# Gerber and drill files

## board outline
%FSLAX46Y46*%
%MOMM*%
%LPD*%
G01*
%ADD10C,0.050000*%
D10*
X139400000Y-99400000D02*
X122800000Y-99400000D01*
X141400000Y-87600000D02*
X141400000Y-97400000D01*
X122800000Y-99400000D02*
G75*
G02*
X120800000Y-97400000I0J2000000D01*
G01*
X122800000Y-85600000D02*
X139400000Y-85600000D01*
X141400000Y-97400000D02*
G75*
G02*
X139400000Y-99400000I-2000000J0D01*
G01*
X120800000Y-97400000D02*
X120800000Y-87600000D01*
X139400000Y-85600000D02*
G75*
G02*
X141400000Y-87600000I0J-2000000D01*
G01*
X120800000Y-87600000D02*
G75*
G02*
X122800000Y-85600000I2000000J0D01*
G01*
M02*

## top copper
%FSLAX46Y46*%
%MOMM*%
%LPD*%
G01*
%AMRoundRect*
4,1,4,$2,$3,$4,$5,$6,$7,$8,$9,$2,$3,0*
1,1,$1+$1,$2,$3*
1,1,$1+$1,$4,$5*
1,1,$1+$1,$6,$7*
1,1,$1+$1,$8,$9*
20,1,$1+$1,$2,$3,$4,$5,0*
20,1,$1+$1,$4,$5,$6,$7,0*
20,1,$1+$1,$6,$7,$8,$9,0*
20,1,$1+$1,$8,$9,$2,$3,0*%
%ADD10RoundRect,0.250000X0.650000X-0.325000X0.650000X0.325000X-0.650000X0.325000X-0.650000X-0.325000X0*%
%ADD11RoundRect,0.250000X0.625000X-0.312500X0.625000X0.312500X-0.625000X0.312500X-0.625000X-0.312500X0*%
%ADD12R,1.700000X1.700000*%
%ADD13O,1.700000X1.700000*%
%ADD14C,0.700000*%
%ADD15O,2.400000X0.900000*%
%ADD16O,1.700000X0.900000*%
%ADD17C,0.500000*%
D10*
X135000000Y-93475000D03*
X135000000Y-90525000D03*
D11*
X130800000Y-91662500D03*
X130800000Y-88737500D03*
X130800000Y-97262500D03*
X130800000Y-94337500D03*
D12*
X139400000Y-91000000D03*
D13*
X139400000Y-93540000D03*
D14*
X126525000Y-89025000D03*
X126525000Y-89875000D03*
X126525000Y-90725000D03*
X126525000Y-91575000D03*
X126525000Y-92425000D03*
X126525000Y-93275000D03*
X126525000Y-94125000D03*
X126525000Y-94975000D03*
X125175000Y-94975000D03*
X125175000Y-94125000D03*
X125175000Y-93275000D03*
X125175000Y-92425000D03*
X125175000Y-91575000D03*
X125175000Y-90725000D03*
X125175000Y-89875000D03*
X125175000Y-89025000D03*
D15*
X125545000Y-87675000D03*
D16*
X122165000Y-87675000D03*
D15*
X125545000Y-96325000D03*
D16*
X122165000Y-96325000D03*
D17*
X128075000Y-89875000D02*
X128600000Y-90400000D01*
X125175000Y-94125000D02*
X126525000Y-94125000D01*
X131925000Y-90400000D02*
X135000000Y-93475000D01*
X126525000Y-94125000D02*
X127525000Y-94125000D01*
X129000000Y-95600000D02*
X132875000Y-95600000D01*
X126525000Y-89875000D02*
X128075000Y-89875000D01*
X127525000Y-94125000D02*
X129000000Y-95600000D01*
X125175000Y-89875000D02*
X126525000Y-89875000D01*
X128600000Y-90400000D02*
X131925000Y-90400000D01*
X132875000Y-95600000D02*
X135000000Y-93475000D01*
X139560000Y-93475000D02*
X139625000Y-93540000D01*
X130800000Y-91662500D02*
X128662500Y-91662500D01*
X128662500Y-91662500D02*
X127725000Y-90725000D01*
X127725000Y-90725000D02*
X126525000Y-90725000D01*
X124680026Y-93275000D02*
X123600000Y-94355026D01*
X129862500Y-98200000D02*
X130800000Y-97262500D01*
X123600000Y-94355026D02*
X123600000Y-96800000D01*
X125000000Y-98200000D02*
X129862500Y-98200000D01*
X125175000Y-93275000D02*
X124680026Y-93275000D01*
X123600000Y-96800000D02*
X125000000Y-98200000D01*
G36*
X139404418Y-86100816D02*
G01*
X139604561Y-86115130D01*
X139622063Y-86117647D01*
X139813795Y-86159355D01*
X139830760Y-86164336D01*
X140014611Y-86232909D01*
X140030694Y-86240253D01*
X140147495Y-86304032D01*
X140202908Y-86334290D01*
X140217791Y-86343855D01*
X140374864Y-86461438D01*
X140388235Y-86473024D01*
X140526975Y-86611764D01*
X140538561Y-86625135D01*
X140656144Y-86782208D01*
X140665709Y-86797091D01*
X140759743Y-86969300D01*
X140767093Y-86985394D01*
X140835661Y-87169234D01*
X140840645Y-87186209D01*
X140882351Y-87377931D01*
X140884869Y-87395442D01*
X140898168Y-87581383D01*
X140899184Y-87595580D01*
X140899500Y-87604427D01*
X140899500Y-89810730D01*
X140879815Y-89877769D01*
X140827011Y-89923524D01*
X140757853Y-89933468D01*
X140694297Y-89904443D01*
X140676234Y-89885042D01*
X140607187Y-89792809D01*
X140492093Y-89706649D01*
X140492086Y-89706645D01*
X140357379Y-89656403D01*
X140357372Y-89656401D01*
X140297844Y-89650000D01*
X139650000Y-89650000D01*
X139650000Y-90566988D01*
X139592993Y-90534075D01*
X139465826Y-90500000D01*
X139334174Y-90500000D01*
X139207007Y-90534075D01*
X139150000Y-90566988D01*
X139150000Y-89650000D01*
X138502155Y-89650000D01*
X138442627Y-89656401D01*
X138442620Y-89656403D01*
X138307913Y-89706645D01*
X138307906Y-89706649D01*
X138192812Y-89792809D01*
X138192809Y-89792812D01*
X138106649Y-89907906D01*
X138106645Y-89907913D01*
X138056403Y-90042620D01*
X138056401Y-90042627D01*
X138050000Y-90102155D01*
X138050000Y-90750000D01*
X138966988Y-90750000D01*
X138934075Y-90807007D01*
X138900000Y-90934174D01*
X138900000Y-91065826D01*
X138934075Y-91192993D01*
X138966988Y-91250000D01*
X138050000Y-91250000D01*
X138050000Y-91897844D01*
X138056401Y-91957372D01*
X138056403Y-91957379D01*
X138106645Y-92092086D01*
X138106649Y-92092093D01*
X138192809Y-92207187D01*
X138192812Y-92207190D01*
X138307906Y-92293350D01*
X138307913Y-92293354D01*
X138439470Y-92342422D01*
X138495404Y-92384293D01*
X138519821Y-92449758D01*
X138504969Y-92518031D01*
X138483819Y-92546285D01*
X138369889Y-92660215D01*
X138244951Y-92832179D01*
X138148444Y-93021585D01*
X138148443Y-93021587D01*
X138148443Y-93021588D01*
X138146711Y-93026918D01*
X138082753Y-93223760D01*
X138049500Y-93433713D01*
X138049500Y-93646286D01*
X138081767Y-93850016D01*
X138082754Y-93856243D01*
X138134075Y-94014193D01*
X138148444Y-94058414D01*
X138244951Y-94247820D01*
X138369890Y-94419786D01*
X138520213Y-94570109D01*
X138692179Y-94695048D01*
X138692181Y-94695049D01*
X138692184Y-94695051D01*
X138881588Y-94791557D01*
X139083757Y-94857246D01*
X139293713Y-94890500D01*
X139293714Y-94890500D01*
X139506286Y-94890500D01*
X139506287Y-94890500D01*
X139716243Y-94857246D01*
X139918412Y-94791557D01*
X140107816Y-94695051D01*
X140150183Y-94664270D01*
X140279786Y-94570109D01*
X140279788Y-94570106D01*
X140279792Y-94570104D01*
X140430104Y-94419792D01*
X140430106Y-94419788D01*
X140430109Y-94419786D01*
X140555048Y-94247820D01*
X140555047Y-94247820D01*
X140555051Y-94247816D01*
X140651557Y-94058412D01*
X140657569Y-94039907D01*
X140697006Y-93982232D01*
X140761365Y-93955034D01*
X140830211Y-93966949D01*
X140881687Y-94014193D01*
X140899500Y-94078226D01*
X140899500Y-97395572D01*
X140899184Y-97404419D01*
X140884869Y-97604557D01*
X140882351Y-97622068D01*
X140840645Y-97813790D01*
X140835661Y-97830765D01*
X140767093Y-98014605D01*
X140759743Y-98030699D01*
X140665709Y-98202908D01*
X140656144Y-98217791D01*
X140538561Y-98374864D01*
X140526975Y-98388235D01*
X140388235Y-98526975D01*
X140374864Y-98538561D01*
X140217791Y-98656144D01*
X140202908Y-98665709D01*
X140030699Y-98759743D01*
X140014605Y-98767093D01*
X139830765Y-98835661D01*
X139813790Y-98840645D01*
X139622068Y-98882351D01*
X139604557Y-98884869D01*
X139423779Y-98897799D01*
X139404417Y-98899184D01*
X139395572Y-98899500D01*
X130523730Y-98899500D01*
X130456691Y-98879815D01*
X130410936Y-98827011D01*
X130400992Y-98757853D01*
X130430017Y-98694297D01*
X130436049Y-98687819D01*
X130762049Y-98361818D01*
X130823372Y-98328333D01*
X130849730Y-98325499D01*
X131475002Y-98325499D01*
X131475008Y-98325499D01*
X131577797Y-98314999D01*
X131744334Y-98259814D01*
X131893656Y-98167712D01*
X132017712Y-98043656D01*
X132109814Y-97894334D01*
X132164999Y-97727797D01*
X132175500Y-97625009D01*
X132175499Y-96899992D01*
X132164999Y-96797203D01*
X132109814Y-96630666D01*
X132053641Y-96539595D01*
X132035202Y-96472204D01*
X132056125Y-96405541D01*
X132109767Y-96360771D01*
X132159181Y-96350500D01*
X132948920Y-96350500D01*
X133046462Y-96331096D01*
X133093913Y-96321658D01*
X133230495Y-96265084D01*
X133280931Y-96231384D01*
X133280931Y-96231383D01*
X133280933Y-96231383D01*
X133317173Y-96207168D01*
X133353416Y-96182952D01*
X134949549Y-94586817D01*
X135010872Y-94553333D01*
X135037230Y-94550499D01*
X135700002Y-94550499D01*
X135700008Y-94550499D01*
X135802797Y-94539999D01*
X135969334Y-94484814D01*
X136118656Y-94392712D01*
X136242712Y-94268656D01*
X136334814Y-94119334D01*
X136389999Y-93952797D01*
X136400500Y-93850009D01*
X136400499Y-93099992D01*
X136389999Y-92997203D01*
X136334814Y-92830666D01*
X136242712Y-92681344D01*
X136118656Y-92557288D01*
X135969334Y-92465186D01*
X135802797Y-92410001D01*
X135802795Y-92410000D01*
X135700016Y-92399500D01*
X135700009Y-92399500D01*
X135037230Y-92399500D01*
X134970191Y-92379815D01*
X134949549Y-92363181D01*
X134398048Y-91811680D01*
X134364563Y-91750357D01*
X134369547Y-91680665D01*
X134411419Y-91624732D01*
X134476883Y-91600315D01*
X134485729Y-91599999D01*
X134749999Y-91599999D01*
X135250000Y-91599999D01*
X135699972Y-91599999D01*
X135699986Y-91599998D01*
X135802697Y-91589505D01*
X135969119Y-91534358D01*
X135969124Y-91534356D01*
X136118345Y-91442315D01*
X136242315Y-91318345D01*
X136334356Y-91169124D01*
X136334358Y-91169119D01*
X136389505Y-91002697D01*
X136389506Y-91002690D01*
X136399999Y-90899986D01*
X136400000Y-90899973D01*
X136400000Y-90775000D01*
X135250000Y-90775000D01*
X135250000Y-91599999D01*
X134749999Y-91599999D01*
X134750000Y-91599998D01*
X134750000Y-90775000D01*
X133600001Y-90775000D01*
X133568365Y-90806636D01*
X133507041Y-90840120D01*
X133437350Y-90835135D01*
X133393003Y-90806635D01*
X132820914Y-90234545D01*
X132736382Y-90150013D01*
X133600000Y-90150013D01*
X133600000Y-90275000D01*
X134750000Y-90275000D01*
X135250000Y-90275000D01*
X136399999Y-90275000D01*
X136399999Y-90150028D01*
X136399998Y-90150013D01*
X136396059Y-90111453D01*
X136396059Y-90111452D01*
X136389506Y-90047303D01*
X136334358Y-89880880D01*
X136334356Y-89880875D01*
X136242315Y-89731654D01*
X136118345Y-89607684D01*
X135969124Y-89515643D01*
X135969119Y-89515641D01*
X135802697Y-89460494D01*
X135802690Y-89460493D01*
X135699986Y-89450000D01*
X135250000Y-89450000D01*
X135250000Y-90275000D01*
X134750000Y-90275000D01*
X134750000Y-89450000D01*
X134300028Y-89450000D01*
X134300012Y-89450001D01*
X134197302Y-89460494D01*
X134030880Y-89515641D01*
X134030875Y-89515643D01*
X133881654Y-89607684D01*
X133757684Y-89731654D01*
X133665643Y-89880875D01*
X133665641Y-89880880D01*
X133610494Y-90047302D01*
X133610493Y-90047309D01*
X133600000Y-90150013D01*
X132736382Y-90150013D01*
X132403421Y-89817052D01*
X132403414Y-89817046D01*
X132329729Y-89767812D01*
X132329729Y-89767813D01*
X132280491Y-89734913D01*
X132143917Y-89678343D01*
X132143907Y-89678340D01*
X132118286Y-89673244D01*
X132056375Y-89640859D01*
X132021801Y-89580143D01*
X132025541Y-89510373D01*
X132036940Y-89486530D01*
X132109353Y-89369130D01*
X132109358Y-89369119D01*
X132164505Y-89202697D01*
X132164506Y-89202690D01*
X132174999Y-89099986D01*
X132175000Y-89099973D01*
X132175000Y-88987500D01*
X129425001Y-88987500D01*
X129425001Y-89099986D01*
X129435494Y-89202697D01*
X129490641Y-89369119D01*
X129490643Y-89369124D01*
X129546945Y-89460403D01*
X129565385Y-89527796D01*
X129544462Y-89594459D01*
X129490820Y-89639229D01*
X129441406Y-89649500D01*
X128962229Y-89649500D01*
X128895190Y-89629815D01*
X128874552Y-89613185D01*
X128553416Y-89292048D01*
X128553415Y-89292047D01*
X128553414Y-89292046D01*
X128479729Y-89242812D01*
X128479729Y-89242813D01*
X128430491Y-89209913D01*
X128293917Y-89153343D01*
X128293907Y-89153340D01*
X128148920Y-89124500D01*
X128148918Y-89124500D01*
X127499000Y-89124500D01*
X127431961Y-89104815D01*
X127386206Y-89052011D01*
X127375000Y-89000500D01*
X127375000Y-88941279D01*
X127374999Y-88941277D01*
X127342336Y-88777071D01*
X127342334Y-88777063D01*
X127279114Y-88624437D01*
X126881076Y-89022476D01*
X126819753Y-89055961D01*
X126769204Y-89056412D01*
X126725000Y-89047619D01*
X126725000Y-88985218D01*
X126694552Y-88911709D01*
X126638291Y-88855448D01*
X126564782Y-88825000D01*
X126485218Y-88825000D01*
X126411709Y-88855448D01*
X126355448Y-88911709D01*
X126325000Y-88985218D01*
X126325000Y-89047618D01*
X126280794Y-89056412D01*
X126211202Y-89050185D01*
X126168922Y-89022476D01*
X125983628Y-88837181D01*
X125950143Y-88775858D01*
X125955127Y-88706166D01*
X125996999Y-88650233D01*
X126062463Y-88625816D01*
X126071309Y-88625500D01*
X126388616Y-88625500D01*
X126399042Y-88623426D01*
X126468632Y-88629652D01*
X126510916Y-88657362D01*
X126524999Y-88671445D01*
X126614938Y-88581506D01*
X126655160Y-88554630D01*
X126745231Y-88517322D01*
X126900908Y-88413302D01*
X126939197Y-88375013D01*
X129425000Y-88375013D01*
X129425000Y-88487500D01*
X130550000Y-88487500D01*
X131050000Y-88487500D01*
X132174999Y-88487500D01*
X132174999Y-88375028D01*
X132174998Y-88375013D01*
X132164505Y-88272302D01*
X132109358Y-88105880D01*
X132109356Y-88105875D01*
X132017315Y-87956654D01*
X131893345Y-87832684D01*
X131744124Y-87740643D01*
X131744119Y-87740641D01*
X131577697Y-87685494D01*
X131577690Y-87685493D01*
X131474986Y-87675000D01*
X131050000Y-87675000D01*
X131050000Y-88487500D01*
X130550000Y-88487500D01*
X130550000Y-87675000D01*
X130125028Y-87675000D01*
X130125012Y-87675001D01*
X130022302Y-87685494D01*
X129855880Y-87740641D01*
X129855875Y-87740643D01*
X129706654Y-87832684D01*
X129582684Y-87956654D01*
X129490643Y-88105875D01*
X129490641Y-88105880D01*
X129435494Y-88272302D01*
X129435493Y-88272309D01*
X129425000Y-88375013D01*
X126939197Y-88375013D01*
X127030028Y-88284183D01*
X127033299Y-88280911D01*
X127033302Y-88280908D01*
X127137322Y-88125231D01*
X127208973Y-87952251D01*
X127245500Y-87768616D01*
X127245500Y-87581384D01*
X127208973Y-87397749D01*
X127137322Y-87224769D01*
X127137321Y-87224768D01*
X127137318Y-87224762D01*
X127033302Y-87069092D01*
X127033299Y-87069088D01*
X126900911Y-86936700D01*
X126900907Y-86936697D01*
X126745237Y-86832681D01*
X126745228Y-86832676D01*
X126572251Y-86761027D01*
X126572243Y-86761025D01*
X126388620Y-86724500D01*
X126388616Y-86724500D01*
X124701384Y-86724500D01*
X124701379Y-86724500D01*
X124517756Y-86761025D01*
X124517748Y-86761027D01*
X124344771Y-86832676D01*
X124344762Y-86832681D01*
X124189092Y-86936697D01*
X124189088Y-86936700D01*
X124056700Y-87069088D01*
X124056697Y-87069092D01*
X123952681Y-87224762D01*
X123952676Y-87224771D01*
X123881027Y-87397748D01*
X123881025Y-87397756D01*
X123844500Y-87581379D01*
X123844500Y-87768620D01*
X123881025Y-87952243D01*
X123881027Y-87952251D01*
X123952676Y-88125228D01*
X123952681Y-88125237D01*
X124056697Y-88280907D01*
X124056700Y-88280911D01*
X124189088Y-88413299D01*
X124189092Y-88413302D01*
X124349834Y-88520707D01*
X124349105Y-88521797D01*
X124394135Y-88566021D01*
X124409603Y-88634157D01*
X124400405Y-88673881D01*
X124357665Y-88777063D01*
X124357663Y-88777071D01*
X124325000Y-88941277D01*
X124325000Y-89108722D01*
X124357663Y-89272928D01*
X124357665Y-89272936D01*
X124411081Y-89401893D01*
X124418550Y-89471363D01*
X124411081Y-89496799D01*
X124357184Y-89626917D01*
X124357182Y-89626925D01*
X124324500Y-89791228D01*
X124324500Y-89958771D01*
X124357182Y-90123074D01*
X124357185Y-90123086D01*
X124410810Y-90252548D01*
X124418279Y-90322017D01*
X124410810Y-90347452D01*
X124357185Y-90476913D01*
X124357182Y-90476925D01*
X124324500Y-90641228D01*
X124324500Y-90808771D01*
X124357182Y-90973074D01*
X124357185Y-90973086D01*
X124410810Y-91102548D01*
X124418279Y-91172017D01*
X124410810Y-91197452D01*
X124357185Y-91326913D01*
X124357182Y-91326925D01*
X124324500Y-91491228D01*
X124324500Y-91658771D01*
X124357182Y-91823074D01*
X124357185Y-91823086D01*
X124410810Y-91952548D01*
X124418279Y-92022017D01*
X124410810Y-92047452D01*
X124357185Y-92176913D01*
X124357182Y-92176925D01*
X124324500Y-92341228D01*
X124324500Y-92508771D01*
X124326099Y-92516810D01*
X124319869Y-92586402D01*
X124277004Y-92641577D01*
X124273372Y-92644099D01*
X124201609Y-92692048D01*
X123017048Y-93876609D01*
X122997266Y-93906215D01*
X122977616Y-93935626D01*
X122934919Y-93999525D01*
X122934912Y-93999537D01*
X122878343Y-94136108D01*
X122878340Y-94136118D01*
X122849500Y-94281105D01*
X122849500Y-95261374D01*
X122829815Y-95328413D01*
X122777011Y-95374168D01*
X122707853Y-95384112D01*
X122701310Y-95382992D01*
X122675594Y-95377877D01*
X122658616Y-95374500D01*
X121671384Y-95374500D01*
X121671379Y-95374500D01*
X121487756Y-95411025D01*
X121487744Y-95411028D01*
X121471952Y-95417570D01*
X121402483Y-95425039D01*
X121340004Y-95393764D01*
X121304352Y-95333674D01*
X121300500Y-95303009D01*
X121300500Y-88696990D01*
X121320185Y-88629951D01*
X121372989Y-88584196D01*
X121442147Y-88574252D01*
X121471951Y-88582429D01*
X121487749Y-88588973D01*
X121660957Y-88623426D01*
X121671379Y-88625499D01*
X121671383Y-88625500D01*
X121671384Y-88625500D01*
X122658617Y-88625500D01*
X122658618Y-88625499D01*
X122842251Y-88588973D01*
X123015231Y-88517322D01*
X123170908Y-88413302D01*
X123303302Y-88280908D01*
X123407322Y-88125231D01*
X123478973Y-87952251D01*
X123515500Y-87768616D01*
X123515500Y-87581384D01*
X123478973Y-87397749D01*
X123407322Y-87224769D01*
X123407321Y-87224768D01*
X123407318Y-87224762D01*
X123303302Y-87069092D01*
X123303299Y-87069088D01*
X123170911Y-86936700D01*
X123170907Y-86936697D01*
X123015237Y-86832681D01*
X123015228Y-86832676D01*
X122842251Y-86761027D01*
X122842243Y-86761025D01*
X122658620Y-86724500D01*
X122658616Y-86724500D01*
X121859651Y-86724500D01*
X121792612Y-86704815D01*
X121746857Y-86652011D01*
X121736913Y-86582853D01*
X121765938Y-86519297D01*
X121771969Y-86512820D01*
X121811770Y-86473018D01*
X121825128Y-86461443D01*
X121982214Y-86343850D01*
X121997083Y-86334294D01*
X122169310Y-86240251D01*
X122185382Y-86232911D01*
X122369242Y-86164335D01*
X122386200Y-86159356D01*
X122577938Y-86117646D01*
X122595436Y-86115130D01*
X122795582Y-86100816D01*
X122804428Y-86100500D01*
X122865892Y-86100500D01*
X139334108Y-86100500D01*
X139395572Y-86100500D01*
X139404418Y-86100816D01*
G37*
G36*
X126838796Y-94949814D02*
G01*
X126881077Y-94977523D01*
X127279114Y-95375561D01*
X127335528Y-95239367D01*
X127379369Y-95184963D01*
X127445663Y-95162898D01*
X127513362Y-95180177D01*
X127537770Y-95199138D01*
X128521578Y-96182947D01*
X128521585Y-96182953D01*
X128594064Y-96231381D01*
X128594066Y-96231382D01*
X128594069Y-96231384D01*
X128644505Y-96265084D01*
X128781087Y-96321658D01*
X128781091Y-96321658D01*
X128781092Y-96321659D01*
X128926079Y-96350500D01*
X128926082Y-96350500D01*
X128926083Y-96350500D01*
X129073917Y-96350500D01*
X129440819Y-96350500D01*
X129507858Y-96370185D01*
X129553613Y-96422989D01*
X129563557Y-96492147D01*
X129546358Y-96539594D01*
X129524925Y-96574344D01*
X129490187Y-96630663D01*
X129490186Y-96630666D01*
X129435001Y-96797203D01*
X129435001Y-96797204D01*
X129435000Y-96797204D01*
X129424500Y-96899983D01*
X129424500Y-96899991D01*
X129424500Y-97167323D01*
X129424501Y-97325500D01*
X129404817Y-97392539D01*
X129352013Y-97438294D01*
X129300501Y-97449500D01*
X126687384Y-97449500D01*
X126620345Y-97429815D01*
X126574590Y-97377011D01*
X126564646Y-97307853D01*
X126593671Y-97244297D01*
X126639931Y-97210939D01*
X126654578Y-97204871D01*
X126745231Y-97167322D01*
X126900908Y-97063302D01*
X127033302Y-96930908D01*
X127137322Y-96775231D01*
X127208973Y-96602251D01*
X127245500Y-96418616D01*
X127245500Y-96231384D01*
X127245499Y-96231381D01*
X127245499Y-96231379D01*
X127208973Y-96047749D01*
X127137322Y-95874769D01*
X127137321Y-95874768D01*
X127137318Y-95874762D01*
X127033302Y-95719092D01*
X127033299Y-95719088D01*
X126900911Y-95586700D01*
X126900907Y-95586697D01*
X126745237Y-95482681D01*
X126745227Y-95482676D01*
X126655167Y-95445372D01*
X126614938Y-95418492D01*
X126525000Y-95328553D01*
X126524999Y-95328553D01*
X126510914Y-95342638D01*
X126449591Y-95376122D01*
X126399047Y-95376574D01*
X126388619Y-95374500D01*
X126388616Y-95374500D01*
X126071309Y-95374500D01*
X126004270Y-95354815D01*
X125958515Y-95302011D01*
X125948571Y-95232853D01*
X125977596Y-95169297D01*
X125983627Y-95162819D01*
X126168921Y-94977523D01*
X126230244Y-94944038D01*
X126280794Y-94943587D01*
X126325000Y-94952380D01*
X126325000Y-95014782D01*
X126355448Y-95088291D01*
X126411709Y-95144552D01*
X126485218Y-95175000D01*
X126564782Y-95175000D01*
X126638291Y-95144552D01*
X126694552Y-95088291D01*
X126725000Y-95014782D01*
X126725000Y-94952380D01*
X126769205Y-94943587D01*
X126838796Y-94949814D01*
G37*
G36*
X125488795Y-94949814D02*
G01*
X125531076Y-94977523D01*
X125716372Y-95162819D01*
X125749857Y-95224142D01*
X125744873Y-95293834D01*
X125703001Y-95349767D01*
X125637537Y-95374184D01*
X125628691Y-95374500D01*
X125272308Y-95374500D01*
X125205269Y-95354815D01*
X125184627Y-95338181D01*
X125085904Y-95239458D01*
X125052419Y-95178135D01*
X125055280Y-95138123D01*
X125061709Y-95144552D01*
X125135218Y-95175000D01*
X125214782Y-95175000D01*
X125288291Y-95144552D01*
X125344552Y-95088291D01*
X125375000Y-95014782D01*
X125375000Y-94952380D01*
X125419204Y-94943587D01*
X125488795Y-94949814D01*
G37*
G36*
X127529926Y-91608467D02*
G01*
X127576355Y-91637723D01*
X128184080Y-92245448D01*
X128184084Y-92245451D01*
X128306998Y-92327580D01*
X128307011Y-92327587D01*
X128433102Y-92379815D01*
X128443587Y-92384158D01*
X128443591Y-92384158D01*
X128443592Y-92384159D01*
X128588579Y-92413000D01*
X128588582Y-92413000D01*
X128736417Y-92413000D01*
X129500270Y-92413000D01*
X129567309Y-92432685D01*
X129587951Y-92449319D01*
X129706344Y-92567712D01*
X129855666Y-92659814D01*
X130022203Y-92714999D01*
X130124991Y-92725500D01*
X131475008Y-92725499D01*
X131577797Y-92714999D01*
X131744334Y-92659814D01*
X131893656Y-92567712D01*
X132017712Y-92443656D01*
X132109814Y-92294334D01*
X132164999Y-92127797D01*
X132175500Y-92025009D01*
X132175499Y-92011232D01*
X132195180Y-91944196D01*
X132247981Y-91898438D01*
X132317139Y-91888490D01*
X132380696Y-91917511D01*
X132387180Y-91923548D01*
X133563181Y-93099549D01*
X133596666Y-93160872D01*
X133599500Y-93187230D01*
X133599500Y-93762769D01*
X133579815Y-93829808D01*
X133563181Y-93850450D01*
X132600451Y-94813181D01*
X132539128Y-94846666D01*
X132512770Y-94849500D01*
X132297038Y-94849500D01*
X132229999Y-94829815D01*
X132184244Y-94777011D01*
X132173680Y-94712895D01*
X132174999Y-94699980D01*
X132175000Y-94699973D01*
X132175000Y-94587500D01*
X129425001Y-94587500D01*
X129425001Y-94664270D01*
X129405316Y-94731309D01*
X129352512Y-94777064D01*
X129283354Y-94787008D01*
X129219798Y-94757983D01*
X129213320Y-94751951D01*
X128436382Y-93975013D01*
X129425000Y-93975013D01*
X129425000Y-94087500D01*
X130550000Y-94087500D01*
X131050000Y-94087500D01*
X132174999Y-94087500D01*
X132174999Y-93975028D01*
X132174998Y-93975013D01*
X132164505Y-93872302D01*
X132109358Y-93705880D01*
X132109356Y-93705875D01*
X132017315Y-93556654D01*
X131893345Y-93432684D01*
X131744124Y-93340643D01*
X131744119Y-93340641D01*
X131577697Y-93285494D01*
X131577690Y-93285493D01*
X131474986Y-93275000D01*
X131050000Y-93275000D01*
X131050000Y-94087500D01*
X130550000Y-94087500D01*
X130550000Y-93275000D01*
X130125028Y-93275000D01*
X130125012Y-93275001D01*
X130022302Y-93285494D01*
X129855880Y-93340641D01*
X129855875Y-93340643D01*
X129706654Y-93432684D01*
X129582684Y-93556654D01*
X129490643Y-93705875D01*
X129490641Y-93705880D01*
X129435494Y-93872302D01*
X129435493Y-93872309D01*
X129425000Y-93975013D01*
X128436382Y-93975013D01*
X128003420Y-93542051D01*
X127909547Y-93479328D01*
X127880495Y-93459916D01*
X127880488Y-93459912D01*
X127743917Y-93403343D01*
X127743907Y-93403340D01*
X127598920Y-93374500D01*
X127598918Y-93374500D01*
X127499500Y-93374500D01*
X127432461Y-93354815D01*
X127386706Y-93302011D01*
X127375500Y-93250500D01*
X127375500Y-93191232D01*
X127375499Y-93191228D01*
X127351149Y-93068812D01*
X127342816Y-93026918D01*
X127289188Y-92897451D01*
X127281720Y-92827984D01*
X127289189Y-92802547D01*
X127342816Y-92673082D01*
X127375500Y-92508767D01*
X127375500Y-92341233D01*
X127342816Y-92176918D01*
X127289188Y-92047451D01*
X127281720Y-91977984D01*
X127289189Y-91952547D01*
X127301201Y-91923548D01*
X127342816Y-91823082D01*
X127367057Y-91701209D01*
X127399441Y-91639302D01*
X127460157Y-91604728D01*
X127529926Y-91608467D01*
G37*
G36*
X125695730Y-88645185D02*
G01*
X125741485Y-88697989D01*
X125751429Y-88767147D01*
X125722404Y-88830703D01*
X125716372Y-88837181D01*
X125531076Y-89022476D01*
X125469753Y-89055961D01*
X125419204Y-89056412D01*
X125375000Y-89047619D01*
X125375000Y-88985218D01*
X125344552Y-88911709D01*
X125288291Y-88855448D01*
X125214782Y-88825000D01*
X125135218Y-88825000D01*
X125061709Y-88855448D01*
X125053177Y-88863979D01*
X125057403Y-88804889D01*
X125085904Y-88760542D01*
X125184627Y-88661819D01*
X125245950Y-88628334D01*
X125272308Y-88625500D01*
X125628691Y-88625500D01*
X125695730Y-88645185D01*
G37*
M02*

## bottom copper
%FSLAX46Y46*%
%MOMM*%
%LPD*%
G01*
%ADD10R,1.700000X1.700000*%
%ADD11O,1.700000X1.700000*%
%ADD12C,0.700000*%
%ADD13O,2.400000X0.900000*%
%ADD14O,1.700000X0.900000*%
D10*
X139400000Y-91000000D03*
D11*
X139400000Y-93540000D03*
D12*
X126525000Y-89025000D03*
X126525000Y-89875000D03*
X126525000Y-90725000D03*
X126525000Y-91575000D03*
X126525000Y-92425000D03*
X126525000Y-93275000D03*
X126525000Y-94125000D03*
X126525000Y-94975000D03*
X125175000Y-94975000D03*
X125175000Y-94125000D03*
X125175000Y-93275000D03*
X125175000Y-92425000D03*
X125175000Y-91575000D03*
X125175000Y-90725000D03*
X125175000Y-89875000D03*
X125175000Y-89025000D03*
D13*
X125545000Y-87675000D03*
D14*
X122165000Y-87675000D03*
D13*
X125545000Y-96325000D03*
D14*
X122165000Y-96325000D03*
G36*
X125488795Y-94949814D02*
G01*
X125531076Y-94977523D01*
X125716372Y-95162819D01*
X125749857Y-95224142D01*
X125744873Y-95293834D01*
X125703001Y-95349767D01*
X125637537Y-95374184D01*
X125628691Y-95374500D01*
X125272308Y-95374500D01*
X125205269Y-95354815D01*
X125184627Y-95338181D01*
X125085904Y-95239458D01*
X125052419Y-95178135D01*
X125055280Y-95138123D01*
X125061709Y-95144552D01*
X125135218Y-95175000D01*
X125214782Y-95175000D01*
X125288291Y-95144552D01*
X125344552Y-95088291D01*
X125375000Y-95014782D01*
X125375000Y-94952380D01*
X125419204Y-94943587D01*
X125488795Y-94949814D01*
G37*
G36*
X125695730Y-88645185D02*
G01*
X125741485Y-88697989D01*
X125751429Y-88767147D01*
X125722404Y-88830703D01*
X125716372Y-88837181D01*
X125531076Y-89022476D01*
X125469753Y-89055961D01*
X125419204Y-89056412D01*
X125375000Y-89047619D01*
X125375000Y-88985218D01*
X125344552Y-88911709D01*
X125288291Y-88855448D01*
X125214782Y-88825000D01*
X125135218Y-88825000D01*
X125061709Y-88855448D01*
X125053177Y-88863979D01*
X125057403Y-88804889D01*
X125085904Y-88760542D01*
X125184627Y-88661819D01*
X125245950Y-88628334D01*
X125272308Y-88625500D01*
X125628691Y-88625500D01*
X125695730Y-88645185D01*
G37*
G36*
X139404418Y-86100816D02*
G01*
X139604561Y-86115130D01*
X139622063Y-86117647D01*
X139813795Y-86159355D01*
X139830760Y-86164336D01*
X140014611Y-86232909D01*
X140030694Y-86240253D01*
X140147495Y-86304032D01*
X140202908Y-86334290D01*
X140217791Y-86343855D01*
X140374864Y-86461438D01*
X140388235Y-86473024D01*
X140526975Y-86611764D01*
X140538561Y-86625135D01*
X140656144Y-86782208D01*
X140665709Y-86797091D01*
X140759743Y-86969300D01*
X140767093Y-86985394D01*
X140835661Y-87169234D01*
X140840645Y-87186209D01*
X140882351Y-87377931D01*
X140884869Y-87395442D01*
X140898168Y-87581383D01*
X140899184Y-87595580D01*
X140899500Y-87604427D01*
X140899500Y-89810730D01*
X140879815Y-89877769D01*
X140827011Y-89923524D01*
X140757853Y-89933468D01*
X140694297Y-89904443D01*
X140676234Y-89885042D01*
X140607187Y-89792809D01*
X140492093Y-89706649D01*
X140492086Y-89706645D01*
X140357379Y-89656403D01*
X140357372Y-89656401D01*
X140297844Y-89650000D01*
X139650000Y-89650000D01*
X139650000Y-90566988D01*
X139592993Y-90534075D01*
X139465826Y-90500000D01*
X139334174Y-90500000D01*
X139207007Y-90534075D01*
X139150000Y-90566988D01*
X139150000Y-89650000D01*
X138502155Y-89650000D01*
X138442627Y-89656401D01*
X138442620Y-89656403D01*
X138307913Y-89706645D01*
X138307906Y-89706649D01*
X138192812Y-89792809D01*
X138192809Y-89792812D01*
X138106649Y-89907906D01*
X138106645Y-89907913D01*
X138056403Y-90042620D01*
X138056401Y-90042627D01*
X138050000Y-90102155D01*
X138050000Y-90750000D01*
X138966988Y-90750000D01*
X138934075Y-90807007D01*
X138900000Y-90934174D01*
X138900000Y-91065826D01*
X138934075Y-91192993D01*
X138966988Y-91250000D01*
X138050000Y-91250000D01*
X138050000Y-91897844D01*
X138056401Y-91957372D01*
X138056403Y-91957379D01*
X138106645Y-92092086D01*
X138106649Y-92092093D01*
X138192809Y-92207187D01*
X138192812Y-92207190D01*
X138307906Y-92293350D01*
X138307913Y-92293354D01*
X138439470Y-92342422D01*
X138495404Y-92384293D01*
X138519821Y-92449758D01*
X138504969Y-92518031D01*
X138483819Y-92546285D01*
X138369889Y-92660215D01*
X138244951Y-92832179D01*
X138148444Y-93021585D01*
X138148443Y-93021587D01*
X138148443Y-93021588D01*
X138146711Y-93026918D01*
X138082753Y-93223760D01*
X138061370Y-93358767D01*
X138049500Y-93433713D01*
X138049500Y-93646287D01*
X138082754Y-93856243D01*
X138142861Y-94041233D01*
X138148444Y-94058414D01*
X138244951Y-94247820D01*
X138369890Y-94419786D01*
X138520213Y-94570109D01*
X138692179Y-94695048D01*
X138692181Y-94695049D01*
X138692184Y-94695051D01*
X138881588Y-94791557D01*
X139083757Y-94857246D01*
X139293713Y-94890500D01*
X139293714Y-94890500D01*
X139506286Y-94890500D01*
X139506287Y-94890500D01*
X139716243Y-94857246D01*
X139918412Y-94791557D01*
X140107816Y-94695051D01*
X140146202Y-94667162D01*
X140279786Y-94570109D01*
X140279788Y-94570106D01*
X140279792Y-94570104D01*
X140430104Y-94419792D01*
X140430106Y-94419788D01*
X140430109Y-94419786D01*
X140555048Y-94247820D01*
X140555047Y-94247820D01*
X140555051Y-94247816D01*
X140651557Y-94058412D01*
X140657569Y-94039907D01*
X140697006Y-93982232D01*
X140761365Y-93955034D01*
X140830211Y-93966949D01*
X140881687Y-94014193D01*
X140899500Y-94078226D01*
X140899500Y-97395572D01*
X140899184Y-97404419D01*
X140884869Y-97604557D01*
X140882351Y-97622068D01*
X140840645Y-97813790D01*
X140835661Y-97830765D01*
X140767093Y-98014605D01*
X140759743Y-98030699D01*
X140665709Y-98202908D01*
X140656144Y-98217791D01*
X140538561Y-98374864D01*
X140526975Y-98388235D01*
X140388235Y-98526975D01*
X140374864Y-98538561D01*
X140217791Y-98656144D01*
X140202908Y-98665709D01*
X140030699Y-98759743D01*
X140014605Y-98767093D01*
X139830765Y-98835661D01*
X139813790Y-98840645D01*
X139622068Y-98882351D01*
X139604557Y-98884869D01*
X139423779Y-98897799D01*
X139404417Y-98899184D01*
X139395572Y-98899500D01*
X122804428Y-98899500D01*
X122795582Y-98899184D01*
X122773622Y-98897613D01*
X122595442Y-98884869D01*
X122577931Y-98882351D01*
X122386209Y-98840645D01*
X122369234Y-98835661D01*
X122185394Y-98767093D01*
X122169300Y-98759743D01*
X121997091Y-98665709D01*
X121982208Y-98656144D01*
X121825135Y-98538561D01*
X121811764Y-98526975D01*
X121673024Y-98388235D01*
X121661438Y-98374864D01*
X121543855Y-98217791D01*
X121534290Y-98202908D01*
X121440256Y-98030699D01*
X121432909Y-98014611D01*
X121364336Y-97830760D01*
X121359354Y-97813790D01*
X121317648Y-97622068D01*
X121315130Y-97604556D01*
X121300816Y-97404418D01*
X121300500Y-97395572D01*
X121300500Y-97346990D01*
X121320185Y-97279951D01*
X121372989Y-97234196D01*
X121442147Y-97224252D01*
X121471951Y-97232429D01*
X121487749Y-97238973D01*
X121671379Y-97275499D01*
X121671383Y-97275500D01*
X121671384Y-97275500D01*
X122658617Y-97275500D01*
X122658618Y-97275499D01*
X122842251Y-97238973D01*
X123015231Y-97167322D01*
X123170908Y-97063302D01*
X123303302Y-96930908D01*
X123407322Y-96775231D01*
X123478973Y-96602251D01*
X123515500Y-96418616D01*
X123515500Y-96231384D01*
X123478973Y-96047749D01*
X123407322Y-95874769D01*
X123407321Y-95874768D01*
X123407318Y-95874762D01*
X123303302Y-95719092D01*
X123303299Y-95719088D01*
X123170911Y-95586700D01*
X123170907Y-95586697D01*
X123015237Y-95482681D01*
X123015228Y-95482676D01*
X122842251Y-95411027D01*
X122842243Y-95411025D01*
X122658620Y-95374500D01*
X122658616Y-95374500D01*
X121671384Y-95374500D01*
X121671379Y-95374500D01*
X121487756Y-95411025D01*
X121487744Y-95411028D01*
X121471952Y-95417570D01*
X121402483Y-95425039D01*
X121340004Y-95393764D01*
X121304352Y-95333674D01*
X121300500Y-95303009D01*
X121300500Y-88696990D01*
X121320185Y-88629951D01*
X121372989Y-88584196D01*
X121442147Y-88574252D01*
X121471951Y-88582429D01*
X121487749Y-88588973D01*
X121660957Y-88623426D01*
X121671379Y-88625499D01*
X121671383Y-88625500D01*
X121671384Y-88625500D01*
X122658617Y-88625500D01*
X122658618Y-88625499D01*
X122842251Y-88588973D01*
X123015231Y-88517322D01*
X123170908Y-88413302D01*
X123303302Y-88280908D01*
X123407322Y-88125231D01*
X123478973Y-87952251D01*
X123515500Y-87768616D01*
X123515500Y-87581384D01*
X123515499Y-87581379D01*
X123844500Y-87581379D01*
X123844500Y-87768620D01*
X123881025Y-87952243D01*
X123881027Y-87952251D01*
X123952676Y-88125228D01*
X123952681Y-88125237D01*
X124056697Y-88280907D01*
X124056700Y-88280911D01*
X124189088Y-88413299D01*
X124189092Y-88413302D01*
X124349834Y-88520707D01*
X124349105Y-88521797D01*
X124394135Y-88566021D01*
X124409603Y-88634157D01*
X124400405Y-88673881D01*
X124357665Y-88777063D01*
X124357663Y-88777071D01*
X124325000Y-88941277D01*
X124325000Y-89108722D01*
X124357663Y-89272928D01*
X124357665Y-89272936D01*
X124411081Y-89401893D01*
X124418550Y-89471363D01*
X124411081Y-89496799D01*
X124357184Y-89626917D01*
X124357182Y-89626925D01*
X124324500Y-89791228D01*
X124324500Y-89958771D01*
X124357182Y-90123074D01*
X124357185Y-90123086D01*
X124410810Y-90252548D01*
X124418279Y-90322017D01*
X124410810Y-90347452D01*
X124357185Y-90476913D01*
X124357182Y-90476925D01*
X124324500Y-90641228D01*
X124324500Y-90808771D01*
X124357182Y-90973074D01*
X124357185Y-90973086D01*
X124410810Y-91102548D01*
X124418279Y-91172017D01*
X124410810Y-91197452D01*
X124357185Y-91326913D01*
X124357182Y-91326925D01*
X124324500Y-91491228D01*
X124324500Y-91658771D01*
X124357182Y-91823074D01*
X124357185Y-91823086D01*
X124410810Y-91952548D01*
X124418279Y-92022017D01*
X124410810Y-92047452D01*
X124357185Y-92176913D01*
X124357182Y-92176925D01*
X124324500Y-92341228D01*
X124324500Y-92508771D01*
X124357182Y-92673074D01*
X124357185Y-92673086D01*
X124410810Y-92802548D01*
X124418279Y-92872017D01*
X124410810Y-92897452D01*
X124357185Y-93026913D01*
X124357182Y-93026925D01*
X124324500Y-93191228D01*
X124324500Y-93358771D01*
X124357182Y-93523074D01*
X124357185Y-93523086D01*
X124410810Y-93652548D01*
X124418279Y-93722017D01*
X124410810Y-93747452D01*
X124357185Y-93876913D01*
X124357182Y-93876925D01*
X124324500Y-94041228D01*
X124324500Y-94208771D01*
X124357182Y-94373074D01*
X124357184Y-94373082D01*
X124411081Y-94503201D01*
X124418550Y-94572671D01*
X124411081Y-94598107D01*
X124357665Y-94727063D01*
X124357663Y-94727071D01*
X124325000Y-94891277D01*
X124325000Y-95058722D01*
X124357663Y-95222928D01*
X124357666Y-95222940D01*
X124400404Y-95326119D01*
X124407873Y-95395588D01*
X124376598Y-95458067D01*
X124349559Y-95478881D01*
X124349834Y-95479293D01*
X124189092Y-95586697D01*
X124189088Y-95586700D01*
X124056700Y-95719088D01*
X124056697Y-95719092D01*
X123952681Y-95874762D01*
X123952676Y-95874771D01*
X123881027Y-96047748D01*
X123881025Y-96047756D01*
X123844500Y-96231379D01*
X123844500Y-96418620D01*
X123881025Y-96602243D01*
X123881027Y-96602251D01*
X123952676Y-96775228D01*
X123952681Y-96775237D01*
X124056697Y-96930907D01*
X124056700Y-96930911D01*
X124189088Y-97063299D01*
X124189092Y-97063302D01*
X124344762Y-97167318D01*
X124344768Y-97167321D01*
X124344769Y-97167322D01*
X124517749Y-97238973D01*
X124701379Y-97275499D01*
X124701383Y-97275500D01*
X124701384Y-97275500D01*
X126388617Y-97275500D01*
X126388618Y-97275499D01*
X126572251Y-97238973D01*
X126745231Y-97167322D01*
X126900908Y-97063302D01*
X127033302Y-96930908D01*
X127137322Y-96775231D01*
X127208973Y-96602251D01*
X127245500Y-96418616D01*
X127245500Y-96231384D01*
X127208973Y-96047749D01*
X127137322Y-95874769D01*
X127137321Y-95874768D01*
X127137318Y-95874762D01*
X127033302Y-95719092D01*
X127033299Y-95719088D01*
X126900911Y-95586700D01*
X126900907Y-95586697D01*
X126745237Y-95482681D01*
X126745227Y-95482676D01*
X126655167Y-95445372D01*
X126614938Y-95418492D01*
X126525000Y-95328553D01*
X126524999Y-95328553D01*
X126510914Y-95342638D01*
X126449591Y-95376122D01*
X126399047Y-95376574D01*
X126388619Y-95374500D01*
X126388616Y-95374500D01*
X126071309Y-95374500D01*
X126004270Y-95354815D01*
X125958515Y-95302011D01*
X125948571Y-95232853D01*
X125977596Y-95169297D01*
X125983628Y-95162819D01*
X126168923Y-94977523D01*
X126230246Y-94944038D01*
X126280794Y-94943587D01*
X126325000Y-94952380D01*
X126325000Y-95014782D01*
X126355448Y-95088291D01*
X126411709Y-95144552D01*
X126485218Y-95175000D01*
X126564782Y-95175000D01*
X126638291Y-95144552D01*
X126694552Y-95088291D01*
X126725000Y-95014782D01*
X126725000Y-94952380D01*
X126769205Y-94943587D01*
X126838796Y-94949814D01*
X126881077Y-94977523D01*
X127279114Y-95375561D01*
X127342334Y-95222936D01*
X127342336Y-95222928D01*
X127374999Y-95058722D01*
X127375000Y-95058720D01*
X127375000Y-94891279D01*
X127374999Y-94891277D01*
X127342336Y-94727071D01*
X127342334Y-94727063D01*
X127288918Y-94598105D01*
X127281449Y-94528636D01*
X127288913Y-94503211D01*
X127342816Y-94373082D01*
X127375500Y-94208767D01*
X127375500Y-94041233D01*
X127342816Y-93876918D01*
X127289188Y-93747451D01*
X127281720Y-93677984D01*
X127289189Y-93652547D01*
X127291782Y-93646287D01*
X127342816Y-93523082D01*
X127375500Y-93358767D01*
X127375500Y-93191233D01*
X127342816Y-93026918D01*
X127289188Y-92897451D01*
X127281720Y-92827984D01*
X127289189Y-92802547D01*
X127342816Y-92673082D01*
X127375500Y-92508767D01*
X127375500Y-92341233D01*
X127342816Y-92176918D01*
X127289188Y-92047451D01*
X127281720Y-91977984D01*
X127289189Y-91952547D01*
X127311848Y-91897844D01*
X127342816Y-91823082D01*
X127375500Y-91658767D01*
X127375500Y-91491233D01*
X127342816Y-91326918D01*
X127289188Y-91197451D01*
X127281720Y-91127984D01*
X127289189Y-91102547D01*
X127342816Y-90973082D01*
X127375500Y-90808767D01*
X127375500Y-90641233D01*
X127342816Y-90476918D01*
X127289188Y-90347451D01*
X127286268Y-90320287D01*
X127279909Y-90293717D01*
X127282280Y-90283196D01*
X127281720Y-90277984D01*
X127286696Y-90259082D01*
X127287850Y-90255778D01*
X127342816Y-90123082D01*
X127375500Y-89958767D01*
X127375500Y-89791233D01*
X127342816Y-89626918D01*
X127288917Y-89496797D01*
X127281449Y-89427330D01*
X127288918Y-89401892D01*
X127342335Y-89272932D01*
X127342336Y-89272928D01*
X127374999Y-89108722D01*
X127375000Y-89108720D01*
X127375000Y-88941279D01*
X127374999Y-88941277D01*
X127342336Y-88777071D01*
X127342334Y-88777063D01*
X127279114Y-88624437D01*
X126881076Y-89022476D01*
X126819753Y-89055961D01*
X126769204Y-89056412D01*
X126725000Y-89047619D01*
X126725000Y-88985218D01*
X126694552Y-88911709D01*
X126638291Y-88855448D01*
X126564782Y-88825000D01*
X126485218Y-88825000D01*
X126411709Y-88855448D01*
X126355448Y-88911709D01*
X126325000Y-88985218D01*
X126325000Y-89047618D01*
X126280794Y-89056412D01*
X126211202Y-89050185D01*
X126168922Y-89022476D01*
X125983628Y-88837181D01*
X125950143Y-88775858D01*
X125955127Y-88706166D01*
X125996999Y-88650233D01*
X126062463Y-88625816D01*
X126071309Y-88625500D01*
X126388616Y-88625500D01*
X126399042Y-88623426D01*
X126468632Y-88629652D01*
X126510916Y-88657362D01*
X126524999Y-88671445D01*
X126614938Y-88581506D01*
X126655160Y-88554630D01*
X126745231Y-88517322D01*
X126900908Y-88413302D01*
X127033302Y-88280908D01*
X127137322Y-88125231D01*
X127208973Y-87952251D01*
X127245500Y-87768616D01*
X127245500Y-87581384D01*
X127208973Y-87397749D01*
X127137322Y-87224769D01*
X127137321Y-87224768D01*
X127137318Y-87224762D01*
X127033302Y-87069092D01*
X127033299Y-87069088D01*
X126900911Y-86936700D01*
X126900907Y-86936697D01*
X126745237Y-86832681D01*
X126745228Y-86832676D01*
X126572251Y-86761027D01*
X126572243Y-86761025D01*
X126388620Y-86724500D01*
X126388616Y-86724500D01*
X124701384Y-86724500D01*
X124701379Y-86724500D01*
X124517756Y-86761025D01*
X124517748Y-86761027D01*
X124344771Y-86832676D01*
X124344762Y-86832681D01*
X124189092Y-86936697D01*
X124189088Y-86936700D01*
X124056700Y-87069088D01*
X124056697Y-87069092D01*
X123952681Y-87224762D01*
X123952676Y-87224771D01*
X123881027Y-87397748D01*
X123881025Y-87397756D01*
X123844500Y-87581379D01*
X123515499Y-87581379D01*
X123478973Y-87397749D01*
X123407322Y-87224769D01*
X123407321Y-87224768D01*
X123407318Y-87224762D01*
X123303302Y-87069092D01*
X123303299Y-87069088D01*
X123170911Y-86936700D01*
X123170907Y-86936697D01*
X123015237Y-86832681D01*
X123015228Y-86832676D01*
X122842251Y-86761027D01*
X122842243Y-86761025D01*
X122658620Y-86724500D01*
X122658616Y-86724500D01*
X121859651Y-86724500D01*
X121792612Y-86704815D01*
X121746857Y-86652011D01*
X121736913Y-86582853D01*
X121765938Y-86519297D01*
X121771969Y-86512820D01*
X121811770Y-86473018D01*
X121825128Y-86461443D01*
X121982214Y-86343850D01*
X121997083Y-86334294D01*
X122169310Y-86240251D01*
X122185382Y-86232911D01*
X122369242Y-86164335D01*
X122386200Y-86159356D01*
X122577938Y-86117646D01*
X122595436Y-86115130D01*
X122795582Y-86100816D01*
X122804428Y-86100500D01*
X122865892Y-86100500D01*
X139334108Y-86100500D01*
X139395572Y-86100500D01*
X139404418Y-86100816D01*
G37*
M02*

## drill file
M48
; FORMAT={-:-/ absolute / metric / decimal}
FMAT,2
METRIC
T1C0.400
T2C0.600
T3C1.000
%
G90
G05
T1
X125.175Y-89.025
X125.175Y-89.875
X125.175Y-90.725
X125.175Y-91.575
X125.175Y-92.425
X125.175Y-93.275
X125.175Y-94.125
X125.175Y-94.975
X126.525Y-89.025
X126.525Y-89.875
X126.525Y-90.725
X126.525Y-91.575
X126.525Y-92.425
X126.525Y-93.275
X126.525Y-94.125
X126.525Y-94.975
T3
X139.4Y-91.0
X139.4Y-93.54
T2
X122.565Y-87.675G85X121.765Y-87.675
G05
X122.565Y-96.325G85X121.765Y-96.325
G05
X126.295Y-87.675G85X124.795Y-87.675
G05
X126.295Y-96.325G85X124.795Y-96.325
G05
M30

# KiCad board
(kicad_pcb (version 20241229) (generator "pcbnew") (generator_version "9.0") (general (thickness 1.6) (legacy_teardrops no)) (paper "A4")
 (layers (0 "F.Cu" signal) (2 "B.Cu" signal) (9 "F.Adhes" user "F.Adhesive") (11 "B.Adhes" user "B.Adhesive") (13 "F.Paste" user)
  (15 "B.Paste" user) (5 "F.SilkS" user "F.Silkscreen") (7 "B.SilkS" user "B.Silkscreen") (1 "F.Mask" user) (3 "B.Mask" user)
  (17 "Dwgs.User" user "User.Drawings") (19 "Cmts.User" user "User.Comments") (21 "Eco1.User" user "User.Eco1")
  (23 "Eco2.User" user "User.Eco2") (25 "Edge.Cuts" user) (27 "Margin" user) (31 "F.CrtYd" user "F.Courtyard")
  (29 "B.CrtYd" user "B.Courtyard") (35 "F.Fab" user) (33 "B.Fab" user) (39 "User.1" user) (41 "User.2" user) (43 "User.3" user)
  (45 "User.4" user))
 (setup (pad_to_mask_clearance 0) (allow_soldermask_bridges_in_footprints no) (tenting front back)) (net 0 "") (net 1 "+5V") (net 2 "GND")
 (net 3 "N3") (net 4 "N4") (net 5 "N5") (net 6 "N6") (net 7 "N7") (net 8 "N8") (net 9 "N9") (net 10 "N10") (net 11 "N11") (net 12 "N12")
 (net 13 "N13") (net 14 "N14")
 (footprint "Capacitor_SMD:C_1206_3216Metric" (layer "F.Cu") (at 135 92 90)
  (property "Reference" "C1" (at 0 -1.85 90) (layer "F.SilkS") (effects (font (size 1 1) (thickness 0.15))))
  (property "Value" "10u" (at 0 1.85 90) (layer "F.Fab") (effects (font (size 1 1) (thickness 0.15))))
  (pad "1" smd roundrect (at -1.475 0 90) (size 1.15 1.8) (layers "F.Cu" "F.Mask" "F.Paste") (roundrect_rratio 0.217391) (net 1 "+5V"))
  (pad "2" smd roundrect (at 1.475 0 90) (size 1.15 1.8) (layers "F.Cu" "F.Mask" "F.Paste") (roundrect_rratio 0.217391) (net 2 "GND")))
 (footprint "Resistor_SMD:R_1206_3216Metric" (layer "F.Cu") (at 130.8 90.2 90)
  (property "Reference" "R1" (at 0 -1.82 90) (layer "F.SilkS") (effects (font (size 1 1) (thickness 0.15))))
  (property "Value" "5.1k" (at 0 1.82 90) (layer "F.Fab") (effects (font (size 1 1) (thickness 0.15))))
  (pad "1" smd roundrect (at -1.4625 0 90) (size 1.125 1.75) (layers "F.Cu" "F.Mask" "F.Paste") (roundrect_rratio 0.222222) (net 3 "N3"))
  (pad "2" smd roundrect (at 1.4625 0 90) (size 1.125 1.75) (layers "F.Cu" "F.Mask" "F.Paste") (roundrect_rratio 0.222222) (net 2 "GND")))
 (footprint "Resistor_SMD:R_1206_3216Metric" (layer "F.Cu") (at 130.8 95.8 90)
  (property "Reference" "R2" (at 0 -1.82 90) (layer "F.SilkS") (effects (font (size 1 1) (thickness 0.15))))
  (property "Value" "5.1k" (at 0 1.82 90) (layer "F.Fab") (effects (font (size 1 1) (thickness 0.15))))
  (pad "1" smd roundrect (at -1.4625 0 90) (size 1.125 1.75) (layers "F.Cu" "F.Mask" "F.Paste") (roundrect_rratio 0.222222) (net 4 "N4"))
  (pad "2" smd roundrect (at 1.4625 0 90) (size 1.125 1.75) (layers "F.Cu" "F.Mask" "F.Paste") (roundrect_rratio 0.222222) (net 2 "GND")))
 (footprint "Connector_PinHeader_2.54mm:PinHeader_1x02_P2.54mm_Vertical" (layer "F.Cu") (at 139.4 91)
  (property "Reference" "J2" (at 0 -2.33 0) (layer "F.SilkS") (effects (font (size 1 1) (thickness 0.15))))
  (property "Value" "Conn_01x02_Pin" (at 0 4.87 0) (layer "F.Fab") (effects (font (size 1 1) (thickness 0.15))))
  (pad "1" thru_hole rect (at 0 0) (size 1.7 1.7) (drill 1) (layers "*.Cu" "*.Mask") (remove_unused_layers no) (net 2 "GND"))
  (pad "2" thru_hole oval (at 0 2.54) (size 1.7 1.7) (drill 1) (layers "*.Cu" "*.Mask") (remove_unused_layers no) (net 1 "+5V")))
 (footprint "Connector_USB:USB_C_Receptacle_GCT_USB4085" (layer "F.Cu") (at 126.525 89.025 -90)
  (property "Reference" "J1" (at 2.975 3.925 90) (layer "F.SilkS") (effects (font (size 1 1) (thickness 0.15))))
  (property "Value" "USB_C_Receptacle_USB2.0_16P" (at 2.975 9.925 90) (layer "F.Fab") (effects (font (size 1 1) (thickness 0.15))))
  (pad "A1" thru_hole circle (at 0 0 270) (size 0.7 0.7) (drill 0.4) (layers "*.Cu" "*.Mask") (remove_unused_layers no) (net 2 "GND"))
  (pad "A4" thru_hole circle (at 0.85 0 270) (size 0.7 0.7) (drill 0.4) (layers "*.Cu" "*.Mask") (remove_unused_layers no) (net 1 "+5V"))
  (pad "A5" thru_hole circle (at 1.7 0 270) (size 0.7 0.7) (drill 0.4) (layers "*.Cu" "*.Mask") (remove_unused_layers no) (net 3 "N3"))
  (pad "A6" thru_hole circle (at 2.55 0 270) (size 0.7 0.7) (drill 0.4) (layers "*.Cu" "*.Mask") (remove_unused_layers no) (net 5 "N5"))
  (pad "A7" thru_hole circle (at 3.4 0 270) (size 0.7 0.7) (drill 0.4) (layers "*.Cu" "*.Mask") (remove_unused_layers no) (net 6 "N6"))
  (pad "A8" thru_hole circle (at 4.25 0 270) (size 0.7 0.7) (drill 0.4) (layers "*.Cu" "*.Mask") (remove_unused_layers no) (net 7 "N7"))
  (pad "A9" thru_hole circle (at 5.1 0 270) (size 0.7 0.7) (drill 0.4) (layers "*.Cu" "*.Mask") (remove_unused_layers no) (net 1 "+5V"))
  (pad "A12" thru_hole circle (at 5.95 0 270) (size 0.7 0.7) (drill 0.4) (layers "*.Cu" "*.Mask") (remove_unused_layers no) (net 2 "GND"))
  (pad "B1" thru_hole circle (at 5.95 1.35 270) (size 0.7 0.7) (drill 0.4) (layers "*.Cu" "*.Mask") (remove_unused_layers no) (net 2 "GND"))
  (pad "B4" thru_hole circle (at 5.1 1.35 270) (size 0.7 0.7) (drill 0.4) (layers "*.Cu" "*.Mask") (remove_unused_layers no) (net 1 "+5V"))
  (pad "B5" thru_hole circle (at 4.25 1.35 270) (size 0.7 0.7) (drill 0.4) (layers "*.Cu" "*.Mask") (remove_unused_layers no) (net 4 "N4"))
  (pad "B6" thru_hole circle (at 3.4 1.35 270) (size 0.7 0.7) (drill 0.4) (layers "*.Cu" "*.Mask") (remove_unused_layers no) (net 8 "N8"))
  (pad "B7" thru_hole circle (at 2.55 1.35 270) (size 0.7 0.7) (drill 0.4) (layers "*.Cu" "*.Mask") (remove_unused_layers no) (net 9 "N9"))
  (pad "B8" thru_hole circle (at 1.7 1.35 270) (size 0.7 0.7) (drill 0.4) (layers "*.Cu" "*.Mask") (remove_unused_layers no) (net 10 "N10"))
  (pad "B9" thru_hole circle (at 0.85 1.35 270) (size 0.7 0.7) (drill 0.4) (layers "*.Cu" "*.Mask") (remove_unused_layers no) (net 1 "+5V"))
  (pad "B12" thru_hole circle (at 0 1.35 270) (size 0.7 0.7) (drill 0.4) (layers "*.Cu" "*.Mask") (remove_unused_layers no) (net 2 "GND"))
  (pad "S1" thru_hole oval (at -1.35 0.98 270) (size 0.9 2.4) (drill oval 0.6 2.1) (layers "*.Cu" "*.Mask") (remove_unused_layers no)
   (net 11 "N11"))
  (pad "S1" thru_hole oval (at -1.35 4.36 270) (size 0.9 1.7) (drill oval 0.6 1.4) (layers "*.Cu" "*.Mask") (remove_unused_layers no)
   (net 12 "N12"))
  (pad "S1" thru_hole oval (at 7.3 0.98 270) (size 0.9 2.4) (drill oval 0.6 2.1) (layers "*.Cu" "*.Mask") (remove_unused_layers no)
   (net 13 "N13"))
  (pad "S1" thru_hole oval (at 7.3 4.36 270) (size 0.9 1.7) (drill oval 0.6 1.4) (layers "*.Cu" "*.Mask") (remove_unused_layers no)
   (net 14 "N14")))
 (gr_line (start 139.4 99.4) (end 122.8 99.4) (stroke (width 0.05) (type default)) (layer "Edge.Cuts"))
 (gr_line (start 141.4 87.6) (end 141.4 97.4) (stroke (width 0.05) (type default)) (layer "Edge.Cuts"))
 (gr_arc (start 122.8 99.4) (mid 121.385786 98.814214) (end 120.8 97.4) (stroke (width 0.05) (type default)) (layer "Edge.Cuts"))
 (gr_line (start 122.8 85.6) (end 139.4 85.6) (stroke (width 0.05) (type default)) (layer "Edge.Cuts"))
 (gr_arc (start 141.4 97.4) (mid 140.814214 98.814214) (end 139.4 99.4) (stroke (width 0.05) (type default)) (layer "Edge.Cuts"))
 (gr_line (start 120.8 97.4) (end 120.8 87.6) (stroke (width 0.05) (type default)) (layer "Edge.Cuts"))
 (gr_arc (start 139.4 85.6) (mid 140.814214 86.185786) (end 141.4 87.6) (stroke (width 0.05) (type default)) (layer "Edge.Cuts"))
 (gr_arc (start 120.8 87.6) (mid 121.385786 86.185786) (end 122.8 85.6) (stroke (width 0.05) (type default)) (layer "Edge.Cuts"))
 (segment (start 128.075 89.875) (end 128.6 90.4) (width 0.5) (layer "F.Cu") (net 1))
 (segment (start 125.175 94.125) (end 126.525 94.125) (width 0.5) (layer "F.Cu") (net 1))
 (segment (start 131.925 90.4) (end 135 93.475) (width 0.5) (layer "F.Cu") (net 1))
 (segment (start 126.525 94.125) (end 127.525 94.125) (width 0.5) (layer "F.Cu") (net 1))
 (segment (start 129 95.6) (end 132.875 95.6) (width 0.5) (layer "F.Cu") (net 1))
 (segment (start 126.525 89.875) (end 128.075 89.875) (width 0.5) (layer "F.Cu") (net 1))
 (segment (start 127.525 94.125) (end 129 95.6) (width 0.5) (layer "F.Cu") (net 1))
 (segment (start 125.175 89.875) (end 126.525 89.875) (width 0.5) (layer "F.Cu") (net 1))
 (segment (start 128.6 90.4) (end 131.925 90.4) (width 0.5) (layer "F.Cu") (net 1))
 (segment (start 132.875 95.6) (end 135 93.475) (width 0.5) (layer "F.Cu") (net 1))
 (segment (start 139.56 93.475) (end 139.625 93.54) (width 0.5) (layer "F.Cu") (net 1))
 (segment (start 130.8 91.6625) (end 128.6625 91.6625) (width 0.5) (layer "F.Cu") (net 3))
 (segment (start 128.6625 91.6625) (end 127.725 90.725) (width 0.5) (layer "F.Cu") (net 3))
 (segment (start 127.725 90.725) (end 126.525 90.725) (width 0.5) (layer "F.Cu") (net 3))
 (segment (start 124.680026 93.275) (end 123.6 94.355026) (width 0.5) (layer "F.Cu") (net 4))
 (segment (start 129.8625 98.2) (end 130.8 97.2625) (width 0.5) (layer "F.Cu") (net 4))
 (segment (start 123.6 94.355026) (end 123.6 96.8) (width 0.5) (layer "F.Cu") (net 4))
 (segment (start 125 98.2) (end 129.8625 98.2) (width 0.5) (layer "F.Cu") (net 4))
 (segment (start 125.175 93.275) (end 124.680026 93.275) (width 0.5) (layer "F.Cu") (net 4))
 (segment (start 123.6 96.8) (end 125 98.2) (width 0.5) (layer "F.Cu") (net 4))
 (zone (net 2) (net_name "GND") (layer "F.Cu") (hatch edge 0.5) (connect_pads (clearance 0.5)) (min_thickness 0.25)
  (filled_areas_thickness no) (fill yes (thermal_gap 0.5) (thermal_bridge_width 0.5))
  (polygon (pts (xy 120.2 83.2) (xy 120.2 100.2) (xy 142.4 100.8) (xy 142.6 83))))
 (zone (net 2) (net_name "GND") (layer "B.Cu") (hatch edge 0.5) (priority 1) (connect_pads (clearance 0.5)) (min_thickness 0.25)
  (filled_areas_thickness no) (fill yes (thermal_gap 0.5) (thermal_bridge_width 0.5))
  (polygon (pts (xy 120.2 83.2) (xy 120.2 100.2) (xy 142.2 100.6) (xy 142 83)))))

